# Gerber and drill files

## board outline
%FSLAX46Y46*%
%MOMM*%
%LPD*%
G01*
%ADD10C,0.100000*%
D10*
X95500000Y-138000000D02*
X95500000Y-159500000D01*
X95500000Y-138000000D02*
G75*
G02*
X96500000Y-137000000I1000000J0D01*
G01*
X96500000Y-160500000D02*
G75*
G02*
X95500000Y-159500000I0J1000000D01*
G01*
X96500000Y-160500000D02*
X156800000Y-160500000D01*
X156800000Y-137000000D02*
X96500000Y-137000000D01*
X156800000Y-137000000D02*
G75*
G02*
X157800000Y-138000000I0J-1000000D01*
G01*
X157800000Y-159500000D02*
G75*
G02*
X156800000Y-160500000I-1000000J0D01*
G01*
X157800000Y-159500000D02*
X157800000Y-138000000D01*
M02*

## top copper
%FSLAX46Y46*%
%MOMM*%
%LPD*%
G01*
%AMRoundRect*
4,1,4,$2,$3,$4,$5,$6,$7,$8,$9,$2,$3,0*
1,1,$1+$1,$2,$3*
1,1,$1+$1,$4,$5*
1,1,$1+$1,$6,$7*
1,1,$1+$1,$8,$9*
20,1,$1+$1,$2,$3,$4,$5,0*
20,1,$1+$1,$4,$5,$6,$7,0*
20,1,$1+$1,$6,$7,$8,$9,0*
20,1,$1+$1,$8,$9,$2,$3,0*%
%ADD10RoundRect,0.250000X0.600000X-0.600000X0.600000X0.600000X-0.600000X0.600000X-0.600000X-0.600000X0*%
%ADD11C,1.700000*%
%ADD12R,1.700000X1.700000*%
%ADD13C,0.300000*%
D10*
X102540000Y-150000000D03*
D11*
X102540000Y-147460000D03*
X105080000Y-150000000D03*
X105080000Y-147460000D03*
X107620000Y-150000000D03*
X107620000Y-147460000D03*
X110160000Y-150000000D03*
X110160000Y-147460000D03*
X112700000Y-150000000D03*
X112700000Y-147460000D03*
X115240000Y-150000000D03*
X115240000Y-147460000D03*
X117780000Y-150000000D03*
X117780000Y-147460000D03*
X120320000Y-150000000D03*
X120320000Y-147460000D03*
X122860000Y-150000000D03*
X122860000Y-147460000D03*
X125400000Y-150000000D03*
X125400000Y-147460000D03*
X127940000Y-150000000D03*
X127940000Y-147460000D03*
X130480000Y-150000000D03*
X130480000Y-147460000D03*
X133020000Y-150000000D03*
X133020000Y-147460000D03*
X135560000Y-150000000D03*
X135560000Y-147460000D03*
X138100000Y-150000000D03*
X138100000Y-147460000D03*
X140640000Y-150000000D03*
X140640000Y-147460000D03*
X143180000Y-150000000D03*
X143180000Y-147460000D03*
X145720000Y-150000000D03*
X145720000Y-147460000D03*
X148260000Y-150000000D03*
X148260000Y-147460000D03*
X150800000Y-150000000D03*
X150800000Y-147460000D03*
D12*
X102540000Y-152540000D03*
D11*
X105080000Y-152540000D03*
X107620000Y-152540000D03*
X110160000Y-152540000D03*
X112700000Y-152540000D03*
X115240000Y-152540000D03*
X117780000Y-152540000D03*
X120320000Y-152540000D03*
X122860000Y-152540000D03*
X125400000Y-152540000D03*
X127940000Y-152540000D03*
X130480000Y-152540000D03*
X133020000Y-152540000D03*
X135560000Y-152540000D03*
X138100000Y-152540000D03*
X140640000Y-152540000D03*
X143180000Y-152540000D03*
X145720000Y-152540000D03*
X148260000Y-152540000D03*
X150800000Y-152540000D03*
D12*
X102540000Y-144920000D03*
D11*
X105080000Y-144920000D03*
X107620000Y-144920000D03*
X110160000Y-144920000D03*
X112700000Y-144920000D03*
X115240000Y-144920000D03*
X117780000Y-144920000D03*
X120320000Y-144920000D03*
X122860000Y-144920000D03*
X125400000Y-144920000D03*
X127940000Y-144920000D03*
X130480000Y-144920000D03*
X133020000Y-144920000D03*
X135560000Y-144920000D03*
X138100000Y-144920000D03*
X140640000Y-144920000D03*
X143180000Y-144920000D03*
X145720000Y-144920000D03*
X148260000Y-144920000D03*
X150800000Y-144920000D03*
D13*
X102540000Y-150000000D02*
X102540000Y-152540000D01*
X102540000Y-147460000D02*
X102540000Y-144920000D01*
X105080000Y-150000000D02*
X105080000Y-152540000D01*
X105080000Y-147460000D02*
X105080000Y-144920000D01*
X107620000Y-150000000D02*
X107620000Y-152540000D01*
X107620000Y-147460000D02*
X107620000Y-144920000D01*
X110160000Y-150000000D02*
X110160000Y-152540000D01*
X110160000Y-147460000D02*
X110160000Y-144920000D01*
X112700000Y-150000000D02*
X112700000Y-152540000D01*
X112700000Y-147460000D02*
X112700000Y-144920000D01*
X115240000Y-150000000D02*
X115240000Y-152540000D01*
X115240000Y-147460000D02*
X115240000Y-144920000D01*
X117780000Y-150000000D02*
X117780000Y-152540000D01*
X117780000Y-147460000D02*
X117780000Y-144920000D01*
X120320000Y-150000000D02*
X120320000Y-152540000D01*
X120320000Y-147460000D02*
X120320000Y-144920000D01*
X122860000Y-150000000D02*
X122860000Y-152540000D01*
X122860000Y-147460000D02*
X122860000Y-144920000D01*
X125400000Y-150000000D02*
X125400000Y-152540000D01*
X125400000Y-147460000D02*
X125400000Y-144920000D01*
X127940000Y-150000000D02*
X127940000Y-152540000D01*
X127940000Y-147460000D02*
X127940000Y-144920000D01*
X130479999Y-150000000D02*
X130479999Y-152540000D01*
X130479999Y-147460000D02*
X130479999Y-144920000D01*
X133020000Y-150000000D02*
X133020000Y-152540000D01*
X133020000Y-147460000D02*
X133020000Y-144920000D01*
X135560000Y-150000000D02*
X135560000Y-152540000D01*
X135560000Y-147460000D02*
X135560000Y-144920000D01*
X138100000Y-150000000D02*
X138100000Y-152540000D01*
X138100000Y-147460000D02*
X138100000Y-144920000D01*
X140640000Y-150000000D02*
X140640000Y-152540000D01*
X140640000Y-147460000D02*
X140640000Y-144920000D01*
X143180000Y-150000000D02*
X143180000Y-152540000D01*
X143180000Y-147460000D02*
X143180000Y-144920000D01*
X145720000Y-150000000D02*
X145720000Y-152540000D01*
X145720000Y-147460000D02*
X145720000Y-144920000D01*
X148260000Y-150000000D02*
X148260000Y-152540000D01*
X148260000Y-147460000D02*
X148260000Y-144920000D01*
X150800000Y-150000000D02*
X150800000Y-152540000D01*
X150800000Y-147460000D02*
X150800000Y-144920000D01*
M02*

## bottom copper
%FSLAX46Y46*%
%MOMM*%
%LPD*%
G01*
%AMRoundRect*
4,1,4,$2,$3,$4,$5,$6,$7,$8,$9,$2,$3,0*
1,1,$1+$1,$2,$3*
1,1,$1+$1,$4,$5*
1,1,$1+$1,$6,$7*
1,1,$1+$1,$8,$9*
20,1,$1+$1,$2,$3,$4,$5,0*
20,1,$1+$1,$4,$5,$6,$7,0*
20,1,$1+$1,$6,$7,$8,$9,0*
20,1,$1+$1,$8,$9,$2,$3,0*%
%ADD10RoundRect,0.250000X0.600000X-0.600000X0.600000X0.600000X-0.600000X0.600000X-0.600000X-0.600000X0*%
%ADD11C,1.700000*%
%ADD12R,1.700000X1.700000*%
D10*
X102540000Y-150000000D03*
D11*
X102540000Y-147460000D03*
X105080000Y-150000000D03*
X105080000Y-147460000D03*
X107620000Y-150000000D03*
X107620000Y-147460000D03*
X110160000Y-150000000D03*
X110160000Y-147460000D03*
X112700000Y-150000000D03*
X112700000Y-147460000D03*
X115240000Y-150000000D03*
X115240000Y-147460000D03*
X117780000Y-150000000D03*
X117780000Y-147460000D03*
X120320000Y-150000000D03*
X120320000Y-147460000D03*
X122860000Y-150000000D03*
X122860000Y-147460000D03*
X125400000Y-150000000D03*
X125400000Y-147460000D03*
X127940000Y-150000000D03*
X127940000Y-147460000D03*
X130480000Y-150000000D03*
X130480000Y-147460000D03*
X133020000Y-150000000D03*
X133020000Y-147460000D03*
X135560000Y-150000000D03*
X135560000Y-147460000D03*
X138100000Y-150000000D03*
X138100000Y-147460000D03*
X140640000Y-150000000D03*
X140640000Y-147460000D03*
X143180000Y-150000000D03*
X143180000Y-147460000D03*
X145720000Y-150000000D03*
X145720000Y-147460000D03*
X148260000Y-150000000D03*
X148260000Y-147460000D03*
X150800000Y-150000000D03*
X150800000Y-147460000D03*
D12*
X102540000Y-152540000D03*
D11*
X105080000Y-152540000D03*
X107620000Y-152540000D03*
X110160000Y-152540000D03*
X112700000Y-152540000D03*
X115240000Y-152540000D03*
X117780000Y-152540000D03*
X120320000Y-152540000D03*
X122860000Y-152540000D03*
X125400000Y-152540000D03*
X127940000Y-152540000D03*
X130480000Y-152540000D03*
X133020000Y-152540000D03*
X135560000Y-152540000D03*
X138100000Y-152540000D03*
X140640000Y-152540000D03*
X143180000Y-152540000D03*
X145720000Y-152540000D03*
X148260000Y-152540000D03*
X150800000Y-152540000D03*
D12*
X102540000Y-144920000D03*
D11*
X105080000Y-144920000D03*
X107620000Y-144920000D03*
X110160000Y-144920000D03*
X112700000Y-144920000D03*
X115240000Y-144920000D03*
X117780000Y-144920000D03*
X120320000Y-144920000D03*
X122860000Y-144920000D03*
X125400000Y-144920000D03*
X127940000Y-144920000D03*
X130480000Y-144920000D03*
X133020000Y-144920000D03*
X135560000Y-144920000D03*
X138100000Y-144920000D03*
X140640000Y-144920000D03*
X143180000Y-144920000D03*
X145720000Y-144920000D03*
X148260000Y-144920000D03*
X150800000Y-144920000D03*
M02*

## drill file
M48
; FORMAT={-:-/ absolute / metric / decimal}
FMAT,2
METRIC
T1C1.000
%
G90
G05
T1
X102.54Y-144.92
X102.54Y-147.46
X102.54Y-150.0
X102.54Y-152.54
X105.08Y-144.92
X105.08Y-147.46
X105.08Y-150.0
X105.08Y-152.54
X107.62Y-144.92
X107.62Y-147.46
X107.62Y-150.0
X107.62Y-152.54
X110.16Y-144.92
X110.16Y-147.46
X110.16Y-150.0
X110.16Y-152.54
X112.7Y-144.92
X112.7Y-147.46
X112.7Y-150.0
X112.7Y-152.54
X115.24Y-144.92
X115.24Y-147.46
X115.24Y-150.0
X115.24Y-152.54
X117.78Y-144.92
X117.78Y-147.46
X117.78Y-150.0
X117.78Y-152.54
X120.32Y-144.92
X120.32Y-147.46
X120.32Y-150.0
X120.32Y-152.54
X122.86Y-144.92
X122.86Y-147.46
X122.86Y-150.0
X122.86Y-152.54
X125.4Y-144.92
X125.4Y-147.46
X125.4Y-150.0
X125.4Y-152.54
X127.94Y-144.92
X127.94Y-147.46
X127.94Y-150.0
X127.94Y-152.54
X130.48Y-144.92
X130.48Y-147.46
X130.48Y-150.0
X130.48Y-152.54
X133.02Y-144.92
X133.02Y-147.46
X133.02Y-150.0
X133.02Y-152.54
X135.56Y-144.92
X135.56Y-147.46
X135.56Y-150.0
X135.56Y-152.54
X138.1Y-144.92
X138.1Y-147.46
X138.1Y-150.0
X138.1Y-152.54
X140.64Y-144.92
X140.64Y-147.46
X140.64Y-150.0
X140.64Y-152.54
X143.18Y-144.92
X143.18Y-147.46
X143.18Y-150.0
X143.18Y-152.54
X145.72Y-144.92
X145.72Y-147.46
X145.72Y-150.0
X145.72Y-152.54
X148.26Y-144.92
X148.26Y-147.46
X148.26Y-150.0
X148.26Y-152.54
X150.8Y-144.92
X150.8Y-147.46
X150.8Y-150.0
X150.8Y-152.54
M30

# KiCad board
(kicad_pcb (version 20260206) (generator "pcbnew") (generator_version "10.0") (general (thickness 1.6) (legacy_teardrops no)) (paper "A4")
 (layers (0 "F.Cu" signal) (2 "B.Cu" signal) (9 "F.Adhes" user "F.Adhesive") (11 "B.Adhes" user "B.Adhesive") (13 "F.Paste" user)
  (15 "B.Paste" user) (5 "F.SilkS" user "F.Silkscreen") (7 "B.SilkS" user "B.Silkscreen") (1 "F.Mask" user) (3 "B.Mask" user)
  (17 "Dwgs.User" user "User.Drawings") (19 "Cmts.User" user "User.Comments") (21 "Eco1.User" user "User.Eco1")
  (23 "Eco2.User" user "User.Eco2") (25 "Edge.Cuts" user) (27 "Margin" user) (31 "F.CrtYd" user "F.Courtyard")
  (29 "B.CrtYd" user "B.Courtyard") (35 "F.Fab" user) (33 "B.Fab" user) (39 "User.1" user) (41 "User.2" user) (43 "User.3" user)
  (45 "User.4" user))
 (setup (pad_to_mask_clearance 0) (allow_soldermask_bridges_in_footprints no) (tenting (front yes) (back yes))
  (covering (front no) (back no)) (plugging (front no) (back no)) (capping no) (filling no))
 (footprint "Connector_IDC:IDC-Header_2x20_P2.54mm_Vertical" (layer "F.Cu") (at 102.54 150 90)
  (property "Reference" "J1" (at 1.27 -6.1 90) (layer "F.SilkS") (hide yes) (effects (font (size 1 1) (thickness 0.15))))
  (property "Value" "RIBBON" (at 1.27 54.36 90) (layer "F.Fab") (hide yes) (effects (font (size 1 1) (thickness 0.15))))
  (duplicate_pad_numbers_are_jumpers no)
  (pad "1" thru_hole roundrect (at 0 0 90) (size 1.7 1.7) (drill 1) (layers "*.Cu" "*.Mask") (remove_unused_layers no)
   (roundrect_rratio 0.147059) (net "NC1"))
  (pad "2" thru_hole circle (at 2.54 0 90) (size 1.7 1.7) (drill 1) (layers "*.Cu" "*.Mask") (remove_unused_layers no) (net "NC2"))
  (pad "3" thru_hole circle (at 0 2.54 90) (size 1.7 1.7) (drill 1) (layers "*.Cu" "*.Mask") (remove_unused_layers no) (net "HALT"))
  (pad "4" thru_hole circle (at 2.54 2.54 90) (size 1.7 1.7) (drill 1) (layers "*.Cu" "*.Mask") (remove_unused_layers no) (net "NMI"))
  (pad "5" thru_hole circle (at 0 5.08 90) (size 1.7 1.7) (drill 1) (layers "*.Cu" "*.Mask") (remove_unused_layers no) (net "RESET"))
  (pad "6" thru_hole circle (at 2.54 5.08 90) (size 1.7 1.7) (drill 1) (layers "*.Cu" "*.Mask") (remove_unused_layers no) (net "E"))
  (pad "7" thru_hole circle (at 0 7.62 90) (size 1.7 1.7) (drill 1) (layers "*.Cu" "*.Mask") (remove_unused_layers no) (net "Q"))
  (pad "8" thru_hole circle (at 2.54 7.62 90) (size 1.7 1.7) (drill 1) (layers "*.Cu" "*.Mask") (remove_unused_layers no) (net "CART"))
  (pad "9" thru_hole circle (at 0 10.16 90) (size 1.7 1.7) (drill 1) (layers "*.Cu" "*.Mask") (remove_unused_layers no) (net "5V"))
  (pad "10" thru_hole circle (at 2.54 10.16 90) (size 1.7 1.7) (drill 1) (layers "*.Cu" "*.Mask") (remove_unused_layers no) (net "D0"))
  (pad "11" thru_hole circle (at 0 12.7 90) (size 1.7 1.7) (drill 1) (layers "*.Cu" "*.Mask") (remove_unused_layers no) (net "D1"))
  (pad "12" thru_hole circle (at 2.54 12.7 90) (size 1.7 1.7) (drill 1) (layers "*.Cu" "*.Mask") (remove_unused_layers no) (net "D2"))
  (pad "13" thru_hole circle (at 0 15.24 90) (size 1.7 1.7) (drill 1) (layers "*.Cu" "*.Mask") (remove_unused_layers no) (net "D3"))
  (pad "14" thru_hole circle (at 2.54 15.24 90) (size 1.7 1.7) (drill 1) (layers "*.Cu" "*.Mask") (remove_unused_layers no) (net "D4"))
  (pad "15" thru_hole circle (at 0 17.78 90) (size 1.7 1.7) (drill 1) (layers "*.Cu" "*.Mask") (remove_unused_layers no) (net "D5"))
  (pad "16" thru_hole circle (at 2.54 17.78 90) (size 1.7 1.7) (drill 1) (layers "*.Cu" "*.Mask") (remove_unused_layers no) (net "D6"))
  (pad "17" thru_hole circle (at 0 20.32 90) (size 1.7 1.7) (drill 1) (layers "*.Cu" "*.Mask") (remove_unused_layers no) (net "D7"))
  (pad "18" thru_hole circle (at 2.54 20.32 90) (size 1.7 1.7) (drill 1) (layers "*.Cu" "*.Mask") (remove_unused_layers no) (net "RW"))
  (pad "19" thru_hole circle (at 0 22.86 90) (size 1.7 1.7) (drill 1) (layers "*.Cu" "*.Mask") (remove_unused_layers no) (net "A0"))
  (pad "20" thru_hole circle (at 2.54 22.86 90) (size 1.7 1.7) (drill 1) (layers "*.Cu" "*.Mask") (remove_unused_layers no) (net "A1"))
  (pad "21" thru_hole circle (at 0 25.4 90) (size 1.7 1.7) (drill 1) (layers "*.Cu" "*.Mask") (remove_unused_layers no) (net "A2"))
  (pad "22" thru_hole circle (at 2.54 25.4 90) (size 1.7 1.7) (drill 1) (layers "*.Cu" "*.Mask") (remove_unused_layers no) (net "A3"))
  (pad "23" thru_hole circle (at 0 27.94 90) (size 1.7 1.7) (drill 1) (layers "*.Cu" "*.Mask") (remove_unused_layers no) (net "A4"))
  (pad "24" thru_hole circle (at 2.54 27.94 90) (size 1.7 1.7) (drill 1) (layers "*.Cu" "*.Mask") (remove_unused_layers no) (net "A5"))
  (pad "25" thru_hole circle (at 0 30.48 90) (size 1.7 1.7) (drill 1) (layers "*.Cu" "*.Mask") (remove_unused_layers no) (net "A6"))
  (pad "26" thru_hole circle (at 2.54 30.48 90) (size 1.7 1.7) (drill 1) (layers "*.Cu" "*.Mask") (remove_unused_layers no) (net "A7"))
  (pad "27" thru_hole circle (at 0 33.02 90) (size 1.7 1.7) (drill 1) (layers "*.Cu" "*.Mask") (remove_unused_layers no) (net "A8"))
  (pad "28" thru_hole circle (at 2.54 33.02 90) (size 1.7 1.7) (drill 1) (layers "*.Cu" "*.Mask") (remove_unused_layers no) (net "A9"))
  (pad "29" thru_hole circle (at 0 35.56 90) (size 1.7 1.7) (drill 1) (layers "*.Cu" "*.Mask") (remove_unused_layers no) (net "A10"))
  (pad "30" thru_hole circle (at 2.54 35.56 90) (size 1.7 1.7) (drill 1) (layers "*.Cu" "*.Mask") (remove_unused_layers no) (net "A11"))
  (pad "31" thru_hole circle (at 0 38.1 90) (size 1.7 1.7) (drill 1) (layers "*.Cu" "*.Mask") (remove_unused_layers no) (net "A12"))
  (pad "32" thru_hole circle (at 2.54 38.1 90) (size 1.7 1.7) (drill 1) (layers "*.Cu" "*.Mask") (remove_unused_layers no) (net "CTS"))
  (pad "33" thru_hole circle (at 0 40.64 90) (size 1.7 1.7) (drill 1) (layers "*.Cu" "*.Mask") (remove_unused_layers no) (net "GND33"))
  (pad "34" thru_hole circle (at 2.54 40.64 90) (size 1.7 1.7) (drill 1) (layers "*.Cu" "*.Mask") (remove_unused_layers no) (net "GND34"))
  (pad "35" thru_hole circle (at 0 43.18 90) (size 1.7 1.7) (drill 1) (layers "*.Cu" "*.Mask") (remove_unused_layers no) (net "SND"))
  (pad "36" thru_hole circle (at 2.54 43.18 90) (size 1.7 1.7) (drill 1) (layers "*.Cu" "*.Mask") (remove_unused_layers no) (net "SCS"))
  (pad "37" thru_hole circle (at 0 45.72 90) (size 1.7 1.7) (drill 1) (layers "*.Cu" "*.Mask") (remove_unused_layers no) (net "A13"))
  (pad "38" thru_hole circle (at 2.54 45.72 90) (size 1.7 1.7) (drill 1) (layers "*.Cu" "*.Mask") (remove_unused_layers no) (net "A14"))
  (pad "39" thru_hole circle (at 0 48.26 90) (size 1.7 1.7) (drill 1) (layers "*.Cu" "*.Mask") (remove_unused_layers no) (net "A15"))
  (pad "40" thru_hole circle (at 2.54 48.26 90) (size 1.7 1.7) (drill 1) (layers "*.Cu" "*.Mask") (remove_unused_layers no) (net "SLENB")))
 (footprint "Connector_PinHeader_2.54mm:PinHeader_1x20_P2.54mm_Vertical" (layer "B.Cu") (at 102.54 152.54 -90)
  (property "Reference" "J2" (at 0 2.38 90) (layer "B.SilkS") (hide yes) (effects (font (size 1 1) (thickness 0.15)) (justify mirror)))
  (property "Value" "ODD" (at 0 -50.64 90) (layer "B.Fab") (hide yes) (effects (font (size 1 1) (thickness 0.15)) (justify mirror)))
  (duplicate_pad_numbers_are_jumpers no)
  (pad "1" thru_hole rect (at 0 0 270) (size 1.7 1.7) (drill 1) (layers "*.Cu" "*.Mask") (remove_unused_layers no) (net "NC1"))
  (pad "2" thru_hole circle (at 0 -2.54 270) (size 1.7 1.7) (drill 1) (layers "*.Cu" "*.Mask") (remove_unused_layers no) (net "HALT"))
  (pad "3" thru_hole circle (at 0 -5.08 270) (size 1.7 1.7) (drill 1) (layers "*.Cu" "*.Mask") (remove_unused_layers no) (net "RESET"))
  (pad "4" thru_hole circle (at 0 -7.62 270) (size 1.7 1.7) (drill 1) (layers "*.Cu" "*.Mask") (remove_unused_layers no) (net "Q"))
  (pad "5" thru_hole circle (at 0 -10.16 270) (size 1.7 1.7) (drill 1) (layers "*.Cu" "*.Mask") (remove_unused_layers no) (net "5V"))
  (pad "6" thru_hole circle (at 0 -12.7 270) (size 1.7 1.7) (drill 1) (layers "*.Cu" "*.Mask") (remove_unused_layers no) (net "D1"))
  (pad "7" thru_hole circle (at 0 -15.24 270) (size 1.7 1.7) (drill 1) (layers "*.Cu" "*.Mask") (remove_unused_layers no) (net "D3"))
  (pad "8" thru_hole circle (at 0 -17.78 270) (size 1.7 1.7) (drill 1) (layers "*.Cu" "*.Mask") (remove_unused_layers no) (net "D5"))
  (pad "9" thru_hole circle (at 0 -20.32 270) (size 1.7 1.7) (drill 1) (layers "*.Cu" "*.Mask") (remove_unused_layers no) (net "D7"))
  (pad "10" thru_hole circle (at 0 -22.86 270) (size 1.7 1.7) (drill 1) (layers "*.Cu" "*.Mask") (remove_unused_layers no) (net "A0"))
  (pad "11" thru_hole circle (at 0 -25.4 270) (size 1.7 1.7) (drill 1) (layers "*.Cu" "*.Mask") (remove_unused_layers no) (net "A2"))
  (pad "12" thru_hole circle (at 0 -27.94 270) (size 1.7 1.7) (drill 1) (layers "*.Cu" "*.Mask") (remove_unused_layers no) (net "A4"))
  (pad "13" thru_hole circle (at 0 -30.48 270) (size 1.7 1.7) (drill 1) (layers "*.Cu" "*.Mask") (remove_unused_layers no) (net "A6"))
  (pad "14" thru_hole circle (at 0 -33.02 270) (size 1.7 1.7) (drill 1) (layers "*.Cu" "*.Mask") (remove_unused_layers no) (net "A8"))
  (pad "15" thru_hole circle (at 0 -35.56 270) (size 1.7 1.7) (drill 1) (layers "*.Cu" "*.Mask") (remove_unused_layers no) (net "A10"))
  (pad "16" thru_hole circle (at 0 -38.1 270) (size 1.7 1.7) (drill 1) (layers "*.Cu" "*.Mask") (remove_unused_layers no) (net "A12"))
  (pad "17" thru_hole circle (at 0 -40.64 270) (size 1.7 1.7) (drill 1) (layers "*.Cu" "*.Mask") (remove_unused_layers no) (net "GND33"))
  (pad "18" thru_hole circle (at 0 -43.18 270) (size 1.7 1.7) (drill 1) (layers "*.Cu" "*.Mask") (remove_unused_layers no) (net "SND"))
  (pad "19" thru_hole circle (at 0 -45.72 270) (size 1.7 1.7) (drill 1) (layers "*.Cu" "*.Mask") (remove_unused_layers no) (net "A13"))
  (pad "20" thru_hole circle (at 0 -48.26 270) (size 1.7 1.7) (drill 1) (layers "*.Cu" "*.Mask") (remove_unused_layers no) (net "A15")))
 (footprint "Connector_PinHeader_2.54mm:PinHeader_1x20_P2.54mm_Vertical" (layer "B.Cu") (at 102.54 144.92 -90)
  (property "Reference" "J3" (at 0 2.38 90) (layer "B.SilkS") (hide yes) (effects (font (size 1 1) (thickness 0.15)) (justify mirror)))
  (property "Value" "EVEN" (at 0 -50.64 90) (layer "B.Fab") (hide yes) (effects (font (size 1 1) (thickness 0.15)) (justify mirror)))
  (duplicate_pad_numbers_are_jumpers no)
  (pad "1" thru_hole rect (at 0 0 270) (size 1.7 1.7) (drill 1) (layers "*.Cu" "*.Mask") (remove_unused_layers no) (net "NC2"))
  (pad "2" thru_hole circle (at 0 -2.54 270) (size 1.7 1.7) (drill 1) (layers "*.Cu" "*.Mask") (remove_unused_layers no) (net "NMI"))
  (pad "3" thru_hole circle (at 0 -5.08 270) (size 1.7 1.7) (drill 1) (layers "*.Cu" "*.Mask") (remove_unused_layers no) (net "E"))
  (pad "4" thru_hole circle (at 0 -7.62 270) (size 1.7 1.7) (drill 1) (layers "*.Cu" "*.Mask") (remove_unused_layers no) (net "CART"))
  (pad "5" thru_hole circle (at 0 -10.16 270) (size 1.7 1.7) (drill 1) (layers "*.Cu" "*.Mask") (remove_unused_layers no) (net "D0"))
  (pad "6" thru_hole circle (at 0 -12.7 270) (size 1.7 1.7) (drill 1) (layers "*.Cu" "*.Mask") (remove_unused_layers no) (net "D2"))
  (pad "7" thru_hole circle (at 0 -15.24 270) (size 1.7 1.7) (drill 1) (layers "*.Cu" "*.Mask") (remove_unused_layers no) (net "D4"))
  (pad "8" thru_hole circle (at 0 -17.78 270) (size 1.7 1.7) (drill 1) (layers "*.Cu" "*.Mask") (remove_unused_layers no) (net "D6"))
  (pad "9" thru_hole circle (at 0 -20.32 270) (size 1.7 1.7) (drill 1) (layers "*.Cu" "*.Mask") (remove_unused_layers no) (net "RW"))
  (pad "10" thru_hole circle (at 0 -22.86 270) (size 1.7 1.7) (drill 1) (layers "*.Cu" "*.Mask") (remove_unused_layers no) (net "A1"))
  (pad "11" thru_hole circle (at 0 -25.4 270) (size 1.7 1.7) (drill 1) (layers "*.Cu" "*.Mask") (remove_unused_layers no) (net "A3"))
  (pad "12" thru_hole circle (at 0 -27.94 270) (size 1.7 1.7) (drill 1) (layers "*.Cu" "*.Mask") (remove_unused_layers no) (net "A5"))
  (pad "13" thru_hole circle (at 0 -30.48 270) (size 1.7 1.7) (drill 1) (layers "*.Cu" "*.Mask") (remove_unused_layers no) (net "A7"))
  (pad "14" thru_hole circle (at 0 -33.02 270) (size 1.7 1.7) (drill 1) (layers "*.Cu" "*.Mask") (remove_unused_layers no) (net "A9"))
  (pad "15" thru_hole circle (at 0 -35.56 270) (size 1.7 1.7) (drill 1) (layers "*.Cu" "*.Mask") (remove_unused_layers no) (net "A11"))
  (pad "16" thru_hole circle (at 0 -38.1 270) (size 1.7 1.7) (drill 1) (layers "*.Cu" "*.Mask") (remove_unused_layers no) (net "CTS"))
  (pad "17" thru_hole circle (at 0 -40.64 270) (size 1.7 1.7) (drill 1) (layers "*.Cu" "*.Mask") (remove_unused_layers no) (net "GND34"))
  (pad "18" thru_hole circle (at 0 -43.18 270) (size 1.7 1.7) (drill 1) (layers "*.Cu" "*.Mask") (remove_unused_layers no) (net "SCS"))
  (pad "19" thru_hole circle (at 0 -45.72 270) (size 1.7 1.7) (drill 1) (layers "*.Cu" "*.Mask") (remove_unused_layers no) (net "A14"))
  (pad "20" thru_hole circle (at 0 -48.26 270) (size 1.7 1.7) (drill 1) (layers "*.Cu" "*.Mask") (remove_unused_layers no) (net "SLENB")))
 (gr_line (start 95.5 138) (end 95.5 159.5) (stroke (width 0.1) (type default)) (layer "Edge.Cuts"))
 (gr_arc (start 95.5 138) (mid 95.792893 137.292893) (end 96.5 137) (stroke (width 0.1) (type default)) (layer "Edge.Cuts"))
 (gr_arc (start 96.5 160.5) (mid 95.792893 160.207107) (end 95.5 159.5) (stroke (width 0.1) (type default)) (layer "Edge.Cuts"))
 (gr_line (start 96.5 160.5) (end 156.8 160.5) (stroke (width 0.1) (type default)) (layer "Edge.Cuts"))
 (gr_line (start 156.8 137) (end 96.5 137) (stroke (width 0.1) (type default)) (layer "Edge.Cuts"))
 (gr_arc (start 156.8 137) (mid 157.507107 137.292893) (end 157.8 138) (stroke (width 0.1) (type default)) (layer "Edge.Cuts"))
 (gr_arc (start 157.8 159.5) (mid 157.507107 160.207107) (end 156.8 160.5) (stroke (width 0.1) (type default)) (layer "Edge.Cuts"))
 (gr_line (start 157.8 159.5) (end 157.8 138) (stroke (width 0.1) (type default)) (layer "Edge.Cuts"))
 (segment (start 102.54 150) (end 102.54 152.54) (width 0.3) (layer "F.Cu") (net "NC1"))
 (segment (start 102.54 147.46) (end 102.54 144.92) (width 0.3) (layer "F.Cu") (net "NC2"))
 (segment (start 105.08 150) (end 105.08 152.54) (width 0.3) (layer "F.Cu") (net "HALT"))
 (segment (start 105.08 147.46) (end 105.08 144.92) (width 0.3) (layer "F.Cu") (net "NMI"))
 (segment (start 107.62 150) (end 107.62 152.54) (width 0.3) (layer "F.Cu") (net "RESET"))
 (segment (start 107.62 147.46) (end 107.62 144.92) (width 0.3) (layer "F.Cu") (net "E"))
 (segment (start 110.16 150) (end 110.16 152.54) (width 0.3) (layer "F.Cu") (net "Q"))
 (segment (start 110.16 147.46) (end 110.16 144.92) (width 0.3) (layer "F.Cu") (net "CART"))
 (segment (start 112.7 150) (end 112.7 152.54) (width 0.3) (layer "F.Cu") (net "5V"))
 (segment (start 112.7 147.46) (end 112.7 144.92) (width 0.3) (layer "F.Cu") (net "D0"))
 (segment (start 115.24 150) (end 115.24 152.54) (width 0.3) (layer "F.Cu") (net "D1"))
 (segment (start 115.24 147.46) (end 115.24 144.92) (width 0.3) (layer "F.Cu") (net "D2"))
 (segment (start 117.78 150) (end 117.78 152.54) (width 0.3) (layer "F.Cu") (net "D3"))
 (segment (start 117.78 147.46) (end 117.78 144.92) (width 0.3) (layer "F.Cu") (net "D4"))
 (segment (start 120.32 150) (end 120.32 152.54) (width 0.3) (layer "F.Cu") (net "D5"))
 (segment (start 120.32 147.46) (end 120.32 144.92) (width 0.3) (layer "F.Cu") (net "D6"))
 (segment (start 122.86 150) (end 122.86 152.54) (width 0.3) (layer "F.Cu") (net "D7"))
 (segment (start 122.86 147.46) (end 122.86 144.92) (width 0.3) (layer "F.Cu") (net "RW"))
 (segment (start 125.4 150) (end 125.4 152.54) (width 0.3) (layer "F.Cu") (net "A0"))
 (segment (start 125.4 147.46) (end 125.4 144.92) (width 0.3) (layer "F.Cu") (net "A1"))
 (segment (start 127.94 150) (end 127.94 152.54) (width 0.3) (layer "F.Cu") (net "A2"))
 (segment (start 127.94 147.46) (end 127.94 144.92) (width 0.3) (layer "F.Cu") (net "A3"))
 (segment (start 130.479999 150) (end 130.479999 152.54) (width 0.3) (layer "F.Cu") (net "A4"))
 (segment (start 130.479999 147.46) (end 130.479999 144.92) (width 0.3) (layer "F.Cu") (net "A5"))
 (segment (start 133.02 150) (end 133.02 152.54) (width 0.3) (layer "F.Cu") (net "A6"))
 (segment (start 133.02 147.46) (end 133.02 144.92) (width 0.3) (layer "F.Cu") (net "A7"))
 (segment (start 135.56 150) (end 135.56 152.54) (width 0.3) (layer "F.Cu") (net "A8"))
 (segment (start 135.56 147.46) (end 135.56 144.92) (width 0.3) (layer "F.Cu") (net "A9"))
 (segment (start 138.1 150) (end 138.1 152.54) (width 0.3) (layer "F.Cu") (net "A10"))
 (segment (start 138.1 147.46) (end 138.1 144.92) (width 0.3) (layer "F.Cu") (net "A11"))
 (segment (start 140.64 150) (end 140.64 152.54) (width 0.3) (layer "F.Cu") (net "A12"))
 (segment (start 140.64 147.46) (end 140.64 144.92) (width 0.3) (layer "F.Cu") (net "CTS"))
 (segment (start 143.18 150) (end 143.18 152.54) (width 0.3) (layer "F.Cu") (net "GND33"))
 (segment (start 143.18 147.46) (end 143.18 144.92) (width 0.3) (layer "F.Cu") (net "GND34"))
 (segment (start 145.72 150) (end 145.72 152.54) (width 0.3) (layer "F.Cu") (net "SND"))
 (segment (start 145.72 147.46) (end 145.72 144.92) (width 0.3) (layer "F.Cu") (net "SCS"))
 (segment (start 148.26 150) (end 148.26 152.54) (width 0.3) (layer "F.Cu") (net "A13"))
 (segment (start 148.26 147.46) (end 148.26 144.92) (width 0.3) (layer "F.Cu") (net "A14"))
 (segment (start 150.8 150) (end 150.8 152.54) (width 0.3) (layer "F.Cu") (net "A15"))
 (segment (start 150.8 147.46) (end 150.8 144.92) (width 0.3) (layer "F.Cu") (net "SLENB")))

